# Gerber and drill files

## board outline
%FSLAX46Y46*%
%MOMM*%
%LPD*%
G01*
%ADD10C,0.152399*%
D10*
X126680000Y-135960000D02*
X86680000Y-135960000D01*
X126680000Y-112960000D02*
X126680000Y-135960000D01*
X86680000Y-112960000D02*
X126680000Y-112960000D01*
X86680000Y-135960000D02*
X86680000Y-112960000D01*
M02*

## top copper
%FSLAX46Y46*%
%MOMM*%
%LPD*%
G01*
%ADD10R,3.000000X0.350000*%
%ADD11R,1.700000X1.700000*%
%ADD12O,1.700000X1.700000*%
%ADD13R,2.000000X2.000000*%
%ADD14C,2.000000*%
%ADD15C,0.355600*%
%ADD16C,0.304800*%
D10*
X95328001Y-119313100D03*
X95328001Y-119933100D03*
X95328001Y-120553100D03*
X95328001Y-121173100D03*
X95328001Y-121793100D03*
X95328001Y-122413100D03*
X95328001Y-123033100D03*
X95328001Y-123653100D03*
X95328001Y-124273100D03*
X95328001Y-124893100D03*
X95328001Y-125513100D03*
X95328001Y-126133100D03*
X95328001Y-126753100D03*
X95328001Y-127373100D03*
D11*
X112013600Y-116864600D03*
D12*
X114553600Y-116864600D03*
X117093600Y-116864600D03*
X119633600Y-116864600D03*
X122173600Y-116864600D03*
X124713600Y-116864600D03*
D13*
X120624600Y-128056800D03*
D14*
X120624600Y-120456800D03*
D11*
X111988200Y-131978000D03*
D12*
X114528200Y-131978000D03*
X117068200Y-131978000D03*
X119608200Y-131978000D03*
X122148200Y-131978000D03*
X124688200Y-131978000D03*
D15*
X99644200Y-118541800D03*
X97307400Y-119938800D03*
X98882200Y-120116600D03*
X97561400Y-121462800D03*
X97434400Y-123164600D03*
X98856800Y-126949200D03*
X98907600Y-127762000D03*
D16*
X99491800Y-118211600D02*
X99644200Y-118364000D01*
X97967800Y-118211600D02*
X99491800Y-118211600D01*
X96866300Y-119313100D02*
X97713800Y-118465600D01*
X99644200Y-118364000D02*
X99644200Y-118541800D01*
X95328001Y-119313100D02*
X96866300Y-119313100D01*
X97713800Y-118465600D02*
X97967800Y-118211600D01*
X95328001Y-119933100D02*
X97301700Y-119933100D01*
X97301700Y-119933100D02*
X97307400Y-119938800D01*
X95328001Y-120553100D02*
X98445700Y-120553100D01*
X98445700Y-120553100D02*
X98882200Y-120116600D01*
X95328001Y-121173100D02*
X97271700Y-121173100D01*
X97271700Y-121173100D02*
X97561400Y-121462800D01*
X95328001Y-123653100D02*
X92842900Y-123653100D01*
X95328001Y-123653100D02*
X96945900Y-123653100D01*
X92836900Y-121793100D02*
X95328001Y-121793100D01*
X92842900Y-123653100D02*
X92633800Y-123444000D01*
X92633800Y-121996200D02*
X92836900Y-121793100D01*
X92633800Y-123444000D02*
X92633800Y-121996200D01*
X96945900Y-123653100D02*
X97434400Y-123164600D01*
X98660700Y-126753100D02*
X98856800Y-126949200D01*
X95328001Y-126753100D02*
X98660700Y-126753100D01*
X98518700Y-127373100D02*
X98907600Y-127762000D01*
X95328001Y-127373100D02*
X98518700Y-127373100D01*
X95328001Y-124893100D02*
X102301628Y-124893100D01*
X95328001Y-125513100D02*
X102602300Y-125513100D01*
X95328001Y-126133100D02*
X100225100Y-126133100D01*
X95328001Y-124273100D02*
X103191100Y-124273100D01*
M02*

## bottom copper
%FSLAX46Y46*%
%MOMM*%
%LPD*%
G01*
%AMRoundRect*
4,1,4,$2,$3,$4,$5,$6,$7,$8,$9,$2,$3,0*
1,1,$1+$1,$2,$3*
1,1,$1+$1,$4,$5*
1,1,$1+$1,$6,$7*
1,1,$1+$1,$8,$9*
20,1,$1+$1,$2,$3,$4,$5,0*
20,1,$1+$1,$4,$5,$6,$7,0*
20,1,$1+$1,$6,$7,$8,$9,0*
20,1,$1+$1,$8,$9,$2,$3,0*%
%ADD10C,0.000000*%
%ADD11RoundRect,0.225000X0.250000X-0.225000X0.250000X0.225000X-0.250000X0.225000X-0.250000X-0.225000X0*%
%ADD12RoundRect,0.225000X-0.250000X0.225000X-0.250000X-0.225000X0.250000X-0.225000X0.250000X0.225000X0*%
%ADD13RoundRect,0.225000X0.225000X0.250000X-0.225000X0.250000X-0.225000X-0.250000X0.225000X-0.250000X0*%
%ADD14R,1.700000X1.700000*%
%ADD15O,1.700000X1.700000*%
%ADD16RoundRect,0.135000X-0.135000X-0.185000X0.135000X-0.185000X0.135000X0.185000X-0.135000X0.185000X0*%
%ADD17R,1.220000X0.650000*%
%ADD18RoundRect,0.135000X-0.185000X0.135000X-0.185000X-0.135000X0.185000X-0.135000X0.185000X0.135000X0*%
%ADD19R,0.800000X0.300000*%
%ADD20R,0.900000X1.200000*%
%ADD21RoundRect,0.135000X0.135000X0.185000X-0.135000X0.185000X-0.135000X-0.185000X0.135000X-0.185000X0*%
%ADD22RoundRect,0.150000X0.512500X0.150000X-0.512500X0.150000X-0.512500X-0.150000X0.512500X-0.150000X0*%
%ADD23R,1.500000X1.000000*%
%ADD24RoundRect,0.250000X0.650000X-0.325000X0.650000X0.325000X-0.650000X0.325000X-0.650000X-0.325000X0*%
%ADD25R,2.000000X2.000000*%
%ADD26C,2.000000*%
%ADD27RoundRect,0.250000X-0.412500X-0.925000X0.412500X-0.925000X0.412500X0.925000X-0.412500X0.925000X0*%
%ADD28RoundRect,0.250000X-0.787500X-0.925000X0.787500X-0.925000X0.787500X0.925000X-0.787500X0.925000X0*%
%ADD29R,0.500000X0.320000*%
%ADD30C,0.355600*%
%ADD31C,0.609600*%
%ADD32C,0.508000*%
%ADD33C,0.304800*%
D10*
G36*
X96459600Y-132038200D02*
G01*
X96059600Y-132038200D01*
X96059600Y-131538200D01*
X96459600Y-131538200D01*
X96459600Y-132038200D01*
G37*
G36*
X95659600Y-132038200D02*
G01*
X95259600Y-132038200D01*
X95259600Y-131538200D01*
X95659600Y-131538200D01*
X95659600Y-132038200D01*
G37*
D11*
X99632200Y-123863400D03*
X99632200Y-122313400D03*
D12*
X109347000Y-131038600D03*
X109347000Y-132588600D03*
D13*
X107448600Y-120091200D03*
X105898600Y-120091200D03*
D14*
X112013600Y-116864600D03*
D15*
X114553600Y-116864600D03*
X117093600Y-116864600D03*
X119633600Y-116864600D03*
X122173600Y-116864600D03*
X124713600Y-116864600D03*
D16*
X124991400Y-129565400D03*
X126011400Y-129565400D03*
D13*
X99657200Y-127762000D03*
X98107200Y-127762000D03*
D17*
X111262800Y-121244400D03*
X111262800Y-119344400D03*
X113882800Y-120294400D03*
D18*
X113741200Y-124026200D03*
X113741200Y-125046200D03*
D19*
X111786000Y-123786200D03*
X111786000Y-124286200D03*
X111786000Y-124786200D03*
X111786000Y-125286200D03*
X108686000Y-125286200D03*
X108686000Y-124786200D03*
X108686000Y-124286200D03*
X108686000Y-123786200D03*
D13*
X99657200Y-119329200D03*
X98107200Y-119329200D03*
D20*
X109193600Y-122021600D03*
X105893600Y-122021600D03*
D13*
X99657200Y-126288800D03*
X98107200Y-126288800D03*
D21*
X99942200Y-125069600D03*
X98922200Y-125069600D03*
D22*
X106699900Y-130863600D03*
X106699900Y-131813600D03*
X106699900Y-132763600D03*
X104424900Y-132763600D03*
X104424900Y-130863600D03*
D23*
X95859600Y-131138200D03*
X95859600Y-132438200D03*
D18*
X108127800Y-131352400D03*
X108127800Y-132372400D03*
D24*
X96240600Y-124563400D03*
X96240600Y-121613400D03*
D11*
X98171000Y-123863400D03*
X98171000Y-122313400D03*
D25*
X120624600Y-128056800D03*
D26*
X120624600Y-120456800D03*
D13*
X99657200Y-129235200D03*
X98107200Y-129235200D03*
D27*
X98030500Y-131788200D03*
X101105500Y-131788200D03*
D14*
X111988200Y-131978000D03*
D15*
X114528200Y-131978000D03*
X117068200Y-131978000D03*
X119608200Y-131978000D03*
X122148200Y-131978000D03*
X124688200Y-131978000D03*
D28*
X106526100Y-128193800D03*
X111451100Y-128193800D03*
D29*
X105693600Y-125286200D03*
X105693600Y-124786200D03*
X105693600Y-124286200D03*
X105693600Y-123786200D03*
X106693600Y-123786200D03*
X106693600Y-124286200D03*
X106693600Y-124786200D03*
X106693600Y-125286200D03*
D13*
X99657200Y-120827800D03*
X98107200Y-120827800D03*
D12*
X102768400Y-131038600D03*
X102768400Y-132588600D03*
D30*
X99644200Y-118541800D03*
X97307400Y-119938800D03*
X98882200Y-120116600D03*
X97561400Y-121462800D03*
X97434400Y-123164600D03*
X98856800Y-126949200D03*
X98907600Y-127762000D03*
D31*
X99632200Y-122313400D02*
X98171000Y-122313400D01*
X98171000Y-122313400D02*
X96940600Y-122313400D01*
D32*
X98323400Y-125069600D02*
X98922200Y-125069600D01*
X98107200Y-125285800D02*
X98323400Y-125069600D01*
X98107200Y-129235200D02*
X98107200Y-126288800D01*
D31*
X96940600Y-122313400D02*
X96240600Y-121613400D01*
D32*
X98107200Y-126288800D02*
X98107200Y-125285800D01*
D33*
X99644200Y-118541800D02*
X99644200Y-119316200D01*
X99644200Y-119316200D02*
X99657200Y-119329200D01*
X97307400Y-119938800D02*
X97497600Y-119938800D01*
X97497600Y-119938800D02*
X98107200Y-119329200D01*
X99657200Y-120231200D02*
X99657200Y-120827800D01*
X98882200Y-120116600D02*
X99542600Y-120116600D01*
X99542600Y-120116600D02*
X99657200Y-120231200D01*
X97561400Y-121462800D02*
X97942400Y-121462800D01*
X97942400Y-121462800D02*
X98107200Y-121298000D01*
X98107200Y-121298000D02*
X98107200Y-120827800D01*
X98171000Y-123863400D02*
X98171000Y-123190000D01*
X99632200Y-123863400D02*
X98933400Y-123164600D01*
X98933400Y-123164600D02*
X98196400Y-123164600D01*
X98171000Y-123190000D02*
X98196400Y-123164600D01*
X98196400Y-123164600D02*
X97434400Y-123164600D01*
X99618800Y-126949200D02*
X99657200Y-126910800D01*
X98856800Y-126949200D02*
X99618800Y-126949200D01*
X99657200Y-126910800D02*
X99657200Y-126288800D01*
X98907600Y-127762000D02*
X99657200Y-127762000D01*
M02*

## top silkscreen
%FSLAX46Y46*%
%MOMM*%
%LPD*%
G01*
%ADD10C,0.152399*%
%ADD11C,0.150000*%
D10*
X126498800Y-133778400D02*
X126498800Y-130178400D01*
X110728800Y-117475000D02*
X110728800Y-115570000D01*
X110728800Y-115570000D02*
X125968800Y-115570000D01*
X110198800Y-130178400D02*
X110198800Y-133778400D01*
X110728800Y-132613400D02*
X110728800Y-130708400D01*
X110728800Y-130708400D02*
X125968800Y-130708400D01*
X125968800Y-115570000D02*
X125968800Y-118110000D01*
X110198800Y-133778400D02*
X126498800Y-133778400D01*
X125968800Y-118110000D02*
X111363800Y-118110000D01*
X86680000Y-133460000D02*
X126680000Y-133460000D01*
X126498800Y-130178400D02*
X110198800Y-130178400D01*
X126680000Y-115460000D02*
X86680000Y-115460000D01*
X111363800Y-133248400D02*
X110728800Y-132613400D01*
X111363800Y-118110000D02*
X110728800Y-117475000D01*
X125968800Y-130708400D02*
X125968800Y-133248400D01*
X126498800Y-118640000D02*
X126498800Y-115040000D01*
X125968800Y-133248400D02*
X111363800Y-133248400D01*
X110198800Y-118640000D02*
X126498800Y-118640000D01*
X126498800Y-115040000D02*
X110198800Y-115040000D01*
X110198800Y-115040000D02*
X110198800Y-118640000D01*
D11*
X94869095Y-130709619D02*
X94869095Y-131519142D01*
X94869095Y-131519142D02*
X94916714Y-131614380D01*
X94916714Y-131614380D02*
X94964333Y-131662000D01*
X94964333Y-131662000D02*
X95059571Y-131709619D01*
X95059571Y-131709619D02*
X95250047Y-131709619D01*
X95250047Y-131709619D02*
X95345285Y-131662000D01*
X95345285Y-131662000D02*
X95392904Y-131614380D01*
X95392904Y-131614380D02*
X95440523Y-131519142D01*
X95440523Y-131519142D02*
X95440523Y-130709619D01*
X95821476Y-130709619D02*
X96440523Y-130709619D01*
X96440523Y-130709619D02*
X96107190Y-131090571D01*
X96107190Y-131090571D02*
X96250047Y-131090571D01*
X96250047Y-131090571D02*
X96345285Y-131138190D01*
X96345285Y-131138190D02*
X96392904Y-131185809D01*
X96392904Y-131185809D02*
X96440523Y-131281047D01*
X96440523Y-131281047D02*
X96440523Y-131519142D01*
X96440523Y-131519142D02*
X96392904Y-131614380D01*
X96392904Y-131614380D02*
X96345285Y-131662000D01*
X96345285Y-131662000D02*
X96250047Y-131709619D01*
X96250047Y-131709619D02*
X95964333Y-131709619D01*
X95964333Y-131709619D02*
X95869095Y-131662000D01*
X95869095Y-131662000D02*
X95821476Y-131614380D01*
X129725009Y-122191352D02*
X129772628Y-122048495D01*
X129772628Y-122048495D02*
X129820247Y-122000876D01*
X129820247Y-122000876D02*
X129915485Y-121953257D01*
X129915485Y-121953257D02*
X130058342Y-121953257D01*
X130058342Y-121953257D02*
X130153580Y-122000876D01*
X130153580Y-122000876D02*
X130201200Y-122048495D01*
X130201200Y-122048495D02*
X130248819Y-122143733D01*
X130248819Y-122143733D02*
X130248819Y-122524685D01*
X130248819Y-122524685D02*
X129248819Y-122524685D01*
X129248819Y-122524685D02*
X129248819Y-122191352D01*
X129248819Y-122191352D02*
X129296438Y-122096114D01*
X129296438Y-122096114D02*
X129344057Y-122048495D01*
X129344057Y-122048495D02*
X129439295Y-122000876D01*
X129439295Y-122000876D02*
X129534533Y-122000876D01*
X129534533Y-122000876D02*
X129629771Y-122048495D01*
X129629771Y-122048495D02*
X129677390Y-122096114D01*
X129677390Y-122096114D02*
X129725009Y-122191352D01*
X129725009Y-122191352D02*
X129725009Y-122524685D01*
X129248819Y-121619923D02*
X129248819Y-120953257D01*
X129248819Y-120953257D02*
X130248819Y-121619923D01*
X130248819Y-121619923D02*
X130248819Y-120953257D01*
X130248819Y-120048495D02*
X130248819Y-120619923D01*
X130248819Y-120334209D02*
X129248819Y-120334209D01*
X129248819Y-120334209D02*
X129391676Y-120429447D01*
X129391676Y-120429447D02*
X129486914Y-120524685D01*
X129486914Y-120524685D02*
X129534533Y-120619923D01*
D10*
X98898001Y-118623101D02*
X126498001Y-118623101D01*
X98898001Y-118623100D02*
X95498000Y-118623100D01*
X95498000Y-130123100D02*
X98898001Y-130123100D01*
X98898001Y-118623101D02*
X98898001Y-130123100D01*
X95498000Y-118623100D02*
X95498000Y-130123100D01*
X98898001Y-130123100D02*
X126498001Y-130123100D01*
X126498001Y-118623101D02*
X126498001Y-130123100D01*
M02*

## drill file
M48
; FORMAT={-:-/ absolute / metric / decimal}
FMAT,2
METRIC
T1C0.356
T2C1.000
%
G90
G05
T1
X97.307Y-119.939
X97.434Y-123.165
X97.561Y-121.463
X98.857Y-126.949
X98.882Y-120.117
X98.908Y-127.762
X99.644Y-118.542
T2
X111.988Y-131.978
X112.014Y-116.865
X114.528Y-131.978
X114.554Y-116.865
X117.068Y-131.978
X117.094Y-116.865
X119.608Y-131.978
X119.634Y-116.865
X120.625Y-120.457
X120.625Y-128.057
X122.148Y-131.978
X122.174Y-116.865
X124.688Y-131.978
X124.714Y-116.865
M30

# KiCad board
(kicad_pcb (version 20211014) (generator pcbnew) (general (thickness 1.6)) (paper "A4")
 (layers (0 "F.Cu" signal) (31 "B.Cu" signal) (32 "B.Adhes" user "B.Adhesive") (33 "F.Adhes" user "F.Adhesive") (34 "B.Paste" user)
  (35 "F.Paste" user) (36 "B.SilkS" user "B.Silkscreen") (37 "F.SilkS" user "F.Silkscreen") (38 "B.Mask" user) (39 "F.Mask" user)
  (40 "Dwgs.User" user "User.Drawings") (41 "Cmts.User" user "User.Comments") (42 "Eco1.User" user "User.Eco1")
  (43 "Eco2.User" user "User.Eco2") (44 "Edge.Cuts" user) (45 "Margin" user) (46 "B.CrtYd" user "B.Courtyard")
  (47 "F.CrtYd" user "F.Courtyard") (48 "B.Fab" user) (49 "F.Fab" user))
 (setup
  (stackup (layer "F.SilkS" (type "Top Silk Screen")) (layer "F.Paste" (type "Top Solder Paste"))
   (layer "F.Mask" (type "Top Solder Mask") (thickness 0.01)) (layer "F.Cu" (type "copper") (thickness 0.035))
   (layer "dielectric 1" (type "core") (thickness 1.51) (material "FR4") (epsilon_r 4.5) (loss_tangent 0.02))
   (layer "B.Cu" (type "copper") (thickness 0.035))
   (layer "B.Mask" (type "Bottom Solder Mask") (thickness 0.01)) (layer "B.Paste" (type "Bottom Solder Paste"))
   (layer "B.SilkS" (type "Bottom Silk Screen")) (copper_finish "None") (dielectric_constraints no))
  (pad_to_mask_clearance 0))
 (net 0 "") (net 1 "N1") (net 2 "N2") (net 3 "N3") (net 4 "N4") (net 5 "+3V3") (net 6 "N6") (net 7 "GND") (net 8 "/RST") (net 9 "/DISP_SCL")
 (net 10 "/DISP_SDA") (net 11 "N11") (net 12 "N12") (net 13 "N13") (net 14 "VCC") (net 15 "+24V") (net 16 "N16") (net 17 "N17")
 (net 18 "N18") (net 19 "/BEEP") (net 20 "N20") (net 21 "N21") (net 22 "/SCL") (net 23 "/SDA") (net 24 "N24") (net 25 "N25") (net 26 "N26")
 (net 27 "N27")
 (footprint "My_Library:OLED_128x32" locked (layer "F.Cu") (at 98.898001 130.1231)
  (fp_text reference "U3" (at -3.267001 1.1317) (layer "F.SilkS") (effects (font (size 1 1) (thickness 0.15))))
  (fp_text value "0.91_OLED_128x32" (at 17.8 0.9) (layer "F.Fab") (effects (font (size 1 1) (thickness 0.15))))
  (fp_line (start 0 -11.499999) (end 27.6 -11.499999) (layer "F.SilkS") (width 0.152399))
  (fp_line (start 0 -11.5) (end -3.400001 -11.5) (layer "F.SilkS") (width 0.152399))
  (fp_line (start -3.400001 0) (end 0 0) (layer "F.SilkS") (width 0.152399))
  (fp_line (start 0 -11.499999) (end 0 0) (layer "F.SilkS") (width 0.152399))
  (fp_line (start -3.400001 -11.5) (end -3.400001 0) (layer "F.SilkS") (width 0.152399))
  (fp_line (start 0 0) (end 27.6 0) (layer "F.SilkS") (width 0.152399))
  (fp_line (start 27.6 -11.499999) (end 27.6 0) (layer "F.SilkS") (width 0.152399))
  (pad "1" smd rect locked (at -3.57 -10.81 90) (size 0.35 3) (layers "F.Cu" "F.Paste" "F.Mask") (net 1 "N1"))
  (pad "2" smd rect locked (at -3.57 -10.19 90) (size 0.35 3) (layers "F.Cu" "F.Paste" "F.Mask") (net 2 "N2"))
  (pad "3" smd rect locked (at -3.57 -9.57 90) (size 0.35 3) (layers "F.Cu" "F.Paste" "F.Mask") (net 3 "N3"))
  (pad "4" smd rect locked (at -3.57 -8.95 90) (size 0.35 3) (layers "F.Cu" "F.Paste" "F.Mask") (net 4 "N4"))
  (pad "5" smd rect locked (at -3.57 -8.33 90) (size 0.35 3) (layers "F.Cu" "F.Paste" "F.Mask") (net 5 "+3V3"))
  (pad "6" smd rect locked (at -3.57 -7.71 90) (size 0.35 3) (layers "F.Cu" "F.Paste" "F.Mask") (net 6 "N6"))
  (pad "7" smd rect locked (at -3.57 -7.09 90) (size 0.35 3) (layers "F.Cu" "F.Paste" "F.Mask") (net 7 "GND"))
  (pad "8" smd rect locked (at -3.57 -6.47 90) (size 0.35 3) (layers "F.Cu" "F.Paste" "F.Mask") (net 5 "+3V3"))
  (pad "9" smd rect locked (at -3.57 -5.85 90) (size 0.35 3) (layers "F.Cu" "F.Paste" "F.Mask") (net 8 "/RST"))
  (pad "10" smd rect locked (at -3.57 -5.23 90) (size 0.35 3) (layers "F.Cu" "F.Paste" "F.Mask") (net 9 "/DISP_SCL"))
  (pad "11" smd rect locked (at -3.57 -4.61 90) (size 0.35 3) (layers "F.Cu" "F.Paste" "F.Mask") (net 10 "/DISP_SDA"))
  (pad "12" smd rect locked (at -3.57 -3.99 90) (size 0.35 3) (layers "F.Cu" "F.Paste" "F.Mask") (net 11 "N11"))
  (pad "13" smd rect locked (at -3.57 -3.37 90) (size 0.35 3) (layers "F.Cu" "F.Paste" "F.Mask") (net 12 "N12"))
  (pad "14" smd rect locked (at -3.57 -2.75 90) (size 0.35 3) (layers "F.Cu" "F.Paste" "F.Mask") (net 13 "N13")))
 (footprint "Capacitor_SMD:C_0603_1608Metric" (layer "B.Cu") (at 99.6322 123.0884 90)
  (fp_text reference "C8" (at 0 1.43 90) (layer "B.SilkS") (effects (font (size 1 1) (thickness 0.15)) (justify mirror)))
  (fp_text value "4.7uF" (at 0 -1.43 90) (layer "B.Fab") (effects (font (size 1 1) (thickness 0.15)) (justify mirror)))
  (pad "1" smd roundrect (at -0.775 0 90) (size 0.9 0.95) (layers "B.Cu" "B.Paste" "B.Mask") (roundrect_rratio 0.25) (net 5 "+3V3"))
  (pad "2" smd roundrect (at 0.775 0 90) (size 0.9 0.95) (layers "B.Cu" "B.Paste" "B.Mask") (roundrect_rratio 0.25) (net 7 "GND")))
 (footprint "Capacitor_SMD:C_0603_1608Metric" (layer "B.Cu") (at 109.347 131.8136 -90)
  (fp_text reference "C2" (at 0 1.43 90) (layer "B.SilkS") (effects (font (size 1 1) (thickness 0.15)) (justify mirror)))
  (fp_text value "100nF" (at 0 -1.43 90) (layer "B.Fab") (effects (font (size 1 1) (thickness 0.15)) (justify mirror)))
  (pad "1" smd roundrect (at -0.775 0 270) (size 0.9 0.95) (layers "B.Cu" "B.Paste" "B.Mask") (roundrect_rratio 0.25) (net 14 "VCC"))
  (pad "2" smd roundrect (at 0.775 0 270) (size 0.9 0.95) (layers "B.Cu" "B.Paste" "B.Mask") (roundrect_rratio 0.25) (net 7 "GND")))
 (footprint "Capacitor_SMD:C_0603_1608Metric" (layer "B.Cu") (at 106.6736 120.0912 180)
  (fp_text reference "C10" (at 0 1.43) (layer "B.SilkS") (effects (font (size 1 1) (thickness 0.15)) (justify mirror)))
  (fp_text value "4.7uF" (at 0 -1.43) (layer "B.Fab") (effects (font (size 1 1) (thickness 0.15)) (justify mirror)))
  (pad "1" smd roundrect (at -0.775 0 180) (size 0.9 0.95) (layers "B.Cu" "B.Paste" "B.Mask") (roundrect_rratio 0.25) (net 7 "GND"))
  (pad "2" smd roundrect (at 0.775 0 180) (size 0.9 0.95) (layers "B.Cu" "B.Paste" "B.Mask") (roundrect_rratio 0.25) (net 8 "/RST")))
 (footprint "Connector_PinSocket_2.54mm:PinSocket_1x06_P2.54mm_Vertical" (layer "B.Cu") (at 112.0136 116.8646 -90)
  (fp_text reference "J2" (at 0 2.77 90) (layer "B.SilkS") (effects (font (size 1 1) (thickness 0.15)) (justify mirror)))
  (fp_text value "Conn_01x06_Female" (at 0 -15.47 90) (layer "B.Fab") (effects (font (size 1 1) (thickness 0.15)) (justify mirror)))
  (pad "1" thru_hole rect (at 0 0 270) (size 1.7 1.7) (drill 1) (layers *.Cu *.Mask) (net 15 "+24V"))
  (pad "2" thru_hole oval (at 0 -2.54 270) (size 1.7 1.7) (drill 1) (layers *.Cu *.Mask) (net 15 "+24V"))
  (pad "3" thru_hole oval (at 0 -5.08 270) (size 1.7 1.7) (drill 1) (layers *.Cu *.Mask) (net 7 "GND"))
  (pad "4" thru_hole oval (at 0 -7.62 270) (size 1.7 1.7) (drill 1) (layers *.Cu *.Mask) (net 7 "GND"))
  (pad "5" thru_hole oval (at 0 -10.16 270) (size 1.7 1.7) (drill 1) (layers *.Cu *.Mask) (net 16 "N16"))
  (pad "6" thru_hole oval (at 0 -12.7 270) (size 1.7 1.7) (drill 1) (layers *.Cu *.Mask) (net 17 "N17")))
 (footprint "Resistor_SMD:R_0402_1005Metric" (layer "B.Cu") (at 125.5014 129.5654)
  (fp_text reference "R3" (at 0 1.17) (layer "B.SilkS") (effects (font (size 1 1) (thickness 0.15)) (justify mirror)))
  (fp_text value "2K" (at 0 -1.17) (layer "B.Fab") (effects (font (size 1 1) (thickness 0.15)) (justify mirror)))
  (pad "1" smd roundrect (at -0.51 0) (size 0.54 0.64) (layers "B.Cu" "B.Paste" "B.Mask") (roundrect_rratio 0.25) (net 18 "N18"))
  (pad "2" smd roundrect (at 0.51 0) (size 0.54 0.64) (layers "B.Cu" "B.Paste" "B.Mask") (roundrect_rratio 0.25) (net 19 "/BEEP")))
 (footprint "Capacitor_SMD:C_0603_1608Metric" (layer "B.Cu") (at 98.8822 127.762 180)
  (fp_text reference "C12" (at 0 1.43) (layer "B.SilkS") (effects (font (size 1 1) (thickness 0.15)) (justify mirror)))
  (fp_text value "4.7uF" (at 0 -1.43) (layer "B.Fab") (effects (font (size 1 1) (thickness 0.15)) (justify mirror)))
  (pad "1" smd roundrect (at -0.775 0 180) (size 0.9 0.95) (layers "B.Cu" "B.Paste" "B.Mask") (roundrect_rratio 0.25) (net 13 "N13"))
  (pad "2" smd roundrect (at 0.775 0 180) (size 0.9 0.95) (layers "B.Cu" "B.Paste" "B.Mask") (roundrect_rratio 0.25) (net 7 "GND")))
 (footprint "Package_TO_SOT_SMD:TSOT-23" (layer "B.Cu") (at 112.5728 120.2944)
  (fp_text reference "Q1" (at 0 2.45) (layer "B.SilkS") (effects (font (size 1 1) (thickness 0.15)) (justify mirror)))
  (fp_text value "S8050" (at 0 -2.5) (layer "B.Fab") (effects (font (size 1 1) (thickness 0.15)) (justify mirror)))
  (pad "1" smd rect (at -1.31 0.95) (size 1.22 0.65) (layers "B.Cu" "B.Paste" "B.Mask") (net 7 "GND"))
  (pad "2" smd rect (at -1.31 -0.95) (size 1.22 0.65) (layers "B.Cu" "B.Paste" "B.Mask") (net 18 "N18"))
  (pad "3" smd rect (at 1.31 0) (size 1.22 0.65) (layers "B.Cu" "B.Paste" "B.Mask") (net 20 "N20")))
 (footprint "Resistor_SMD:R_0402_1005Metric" (layer "B.Cu") (at 113.7412 124.5362 -90)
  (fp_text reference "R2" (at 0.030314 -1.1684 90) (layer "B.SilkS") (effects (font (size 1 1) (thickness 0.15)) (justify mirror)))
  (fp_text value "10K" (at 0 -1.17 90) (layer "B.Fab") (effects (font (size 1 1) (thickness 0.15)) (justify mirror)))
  (pad "1" smd roundrect (at -0.51 0 270) (size 0.54 0.64) (layers "B.Cu" "B.Paste" "B.Mask") (roundrect_rratio 0.25) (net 14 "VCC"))
  (pad "2" smd roundrect (at 0.51 0 270) (size 0.54 0.64) (layers "B.Cu" "B.Paste" "B.Mask") (roundrect_rratio 0.25) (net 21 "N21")))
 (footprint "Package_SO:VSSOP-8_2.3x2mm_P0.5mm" (layer "B.Cu") (at 110.236 124.5362 180)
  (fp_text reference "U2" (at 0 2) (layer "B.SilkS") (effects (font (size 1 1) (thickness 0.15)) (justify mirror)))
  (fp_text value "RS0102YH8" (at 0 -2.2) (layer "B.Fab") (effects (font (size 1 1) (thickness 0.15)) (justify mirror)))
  (pad "1" smd rect (at -1.55 0.75 270) (size 0.3 0.8) (layers "B.Cu" "B.Paste" "B.Mask") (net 14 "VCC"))
  (pad "2" smd rect (at -1.55 0.25 270) (size 0.3 0.8) (layers "B.Cu" "B.Paste" "B.Mask") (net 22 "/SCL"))
  (pad "3" smd rect (at -1.55 -0.25 270) (size 0.3 0.8) (layers "B.Cu" "B.Paste" "B.Mask") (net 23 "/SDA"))
  (pad "4" smd rect (at -1.55 -0.75 270) (size 0.3 0.8) (layers "B.Cu" "B.Paste" "B.Mask") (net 21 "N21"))
  (pad "5" smd rect (at 1.55 -0.75 270) (size 0.3 0.8) (layers "B.Cu" "B.Paste" "B.Mask") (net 7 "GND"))
  (pad "6" smd rect (at 1.55 -0.25 270) (size 0.3 0.8) (layers "B.Cu" "B.Paste" "B.Mask") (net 10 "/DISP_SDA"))
  (pad "7" smd rect (at 1.55 0.25 270) (size 0.3 0.8) (layers "B.Cu" "B.Paste" "B.Mask") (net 9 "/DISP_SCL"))
  (pad "8" smd rect (at 1.55 0.75 270) (size 0.3 0.8) (layers "B.Cu" "B.Paste" "B.Mask") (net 5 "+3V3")))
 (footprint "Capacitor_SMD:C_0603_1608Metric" (layer "B.Cu") (at 98.8822 119.3292 180)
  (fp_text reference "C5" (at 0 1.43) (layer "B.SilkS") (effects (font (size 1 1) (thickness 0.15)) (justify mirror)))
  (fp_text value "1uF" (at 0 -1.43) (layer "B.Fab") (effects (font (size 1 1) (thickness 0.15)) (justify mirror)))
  (pad "1" smd roundrect (at -0.775 0 180) (size 0.9 0.95) (layers "B.Cu" "B.Paste" "B.Mask") (roundrect_rratio 0.25) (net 1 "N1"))
  (pad "2" smd roundrect (at 0.775 0 180) (size 0.9 0.95) (layers "B.Cu" "B.Paste" "B.Mask") (roundrect_rratio 0.25) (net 2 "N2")))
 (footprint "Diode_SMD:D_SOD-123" (layer "B.Cu") (at 107.5436 122.0216 180)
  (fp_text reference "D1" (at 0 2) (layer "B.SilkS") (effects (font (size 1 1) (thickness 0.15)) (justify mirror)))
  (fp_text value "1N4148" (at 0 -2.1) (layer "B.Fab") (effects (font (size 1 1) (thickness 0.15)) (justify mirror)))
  (pad "1" smd rect (at -1.65 0 180) (size 0.9 1.2) (layers "B.Cu" "B.Paste" "B.Mask") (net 5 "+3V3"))
  (pad "2" smd rect (at 1.65 0 180) (size 0.9 1.2) (layers "B.Cu" "B.Paste" "B.Mask") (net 8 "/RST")))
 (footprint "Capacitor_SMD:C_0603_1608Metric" (layer "B.Cu") (at 98.8822 126.2888 180)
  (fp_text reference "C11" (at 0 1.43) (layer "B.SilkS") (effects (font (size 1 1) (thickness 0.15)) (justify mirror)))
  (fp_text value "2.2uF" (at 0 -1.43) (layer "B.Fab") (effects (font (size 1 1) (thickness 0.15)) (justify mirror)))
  (pad "1" smd roundrect (at -0.775 0 180) (size 0.9 0.95) (layers "B.Cu" "B.Paste" "B.Mask") (roundrect_rratio 0.25) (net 12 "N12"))
  (pad "2" smd roundrect (at 0.775 0 180) (size 0.9 0.95) (layers "B.Cu" "B.Paste" "B.Mask") (roundrect_rratio 0.25) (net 7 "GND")))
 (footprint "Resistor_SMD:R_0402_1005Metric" (layer "B.Cu") (at 99.4322 125.0696 180)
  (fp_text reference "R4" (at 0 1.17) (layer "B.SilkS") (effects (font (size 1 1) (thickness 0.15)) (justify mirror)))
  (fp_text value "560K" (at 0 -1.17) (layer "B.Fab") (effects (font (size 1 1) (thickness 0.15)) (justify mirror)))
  (pad "1" smd roundrect (at -0.51 0 180) (size 0.54 0.64) (layers "B.Cu" "B.Paste" "B.Mask") (roundrect_rratio 0.25) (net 11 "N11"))
  (pad "2" smd roundrect (at 0.51 0 180) (size 0.54 0.64) (layers "B.Cu" "B.Paste" "B.Mask") (roundrect_rratio 0.25) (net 7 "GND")))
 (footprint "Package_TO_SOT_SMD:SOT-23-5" (layer "B.Cu") (at 105.5624 131.8136 180)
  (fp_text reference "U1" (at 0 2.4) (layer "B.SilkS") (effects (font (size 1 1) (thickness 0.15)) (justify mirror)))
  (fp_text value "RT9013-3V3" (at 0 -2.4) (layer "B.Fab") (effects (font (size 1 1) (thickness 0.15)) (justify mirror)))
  (pad "1" smd roundrect (at -1.1375 0.95 180) (size 1.325 0.6) (layers "B.Cu" "B.Paste" "B.Mask") (roundrect_rratio 0.25) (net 14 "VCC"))
  (pad "2" smd roundrect (at -1.1375 0 180) (size 1.325 0.6) (layers "B.Cu" "B.Paste" "B.Mask") (roundrect_rratio 0.25) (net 7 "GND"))
  (pad "3" smd roundrect (at -1.1375 -0.95 180) (size 1.325 0.6) (layers "B.Cu" "B.Paste" "B.Mask") (roundrect_rratio 0.25) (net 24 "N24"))
  (pad "4" smd roundrect (at 1.1375 -0.95 180) (size 1.325 0.6) (layers "B.Cu" "B.Paste" "B.Mask") (roundrect_rratio 0.25) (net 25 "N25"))
  (pad "5" smd roundrect (at 1.1375 0.95 180) (size 1.325 0.6) (layers "B.Cu" "B.Paste" "B.Mask") (roundrect_rratio 0.25) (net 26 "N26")))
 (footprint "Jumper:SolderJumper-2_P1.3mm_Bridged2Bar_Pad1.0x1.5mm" (layer "B.Cu") (at 95.8596 131.7882 -90)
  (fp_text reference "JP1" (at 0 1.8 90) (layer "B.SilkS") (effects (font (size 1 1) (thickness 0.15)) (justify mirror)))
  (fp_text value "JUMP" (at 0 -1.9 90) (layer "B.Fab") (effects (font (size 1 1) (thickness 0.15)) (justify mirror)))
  (fp_poly (pts (xy -0.25 -0.2) (xy 0.25 -0.2) (xy 0.25 -0.6) (xy -0.25 -0.6)) (layer "B.Cu") (width 0) (fill solid))
  (fp_poly (pts (xy -0.25 0.6) (xy 0.25 0.6) (xy 0.25 0.2) (xy -0.25 0.2)) (layer "B.Cu") (width 0) (fill solid))
  (pad "1" smd rect (at -0.65 0 270) (size 1 1.5) (layers "B.Cu" "B.Mask") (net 5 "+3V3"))
  (pad "2" smd rect (at 0.65 0 270) (size 1 1.5) (layers "B.Cu" "B.Mask") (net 26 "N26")))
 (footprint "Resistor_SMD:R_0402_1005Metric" (layer "B.Cu") (at 108.1278 131.8624 -90)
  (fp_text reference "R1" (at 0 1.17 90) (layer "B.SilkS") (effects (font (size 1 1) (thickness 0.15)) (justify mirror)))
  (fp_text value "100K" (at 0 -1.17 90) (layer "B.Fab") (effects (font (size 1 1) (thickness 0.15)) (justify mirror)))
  (pad "1" smd roundrect (at -0.51 0 270) (size 0.54 0.64) (layers "B.Cu" "B.Paste" "B.Mask") (roundrect_rratio 0.25) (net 14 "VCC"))
  (pad "2" smd roundrect (at 0.51 0 270) (size 0.54 0.64) (layers "B.Cu" "B.Paste" "B.Mask") (roundrect_rratio 0.25) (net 24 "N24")))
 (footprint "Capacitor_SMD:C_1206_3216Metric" (layer "B.Cu") (at 96.2406 123.0884 90)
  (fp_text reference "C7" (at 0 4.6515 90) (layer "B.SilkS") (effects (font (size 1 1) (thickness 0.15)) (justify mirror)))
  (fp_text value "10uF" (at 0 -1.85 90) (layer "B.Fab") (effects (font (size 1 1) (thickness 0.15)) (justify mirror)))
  (pad "1" smd roundrect (at -1.475 0 90) (size 1.15 1.8) (layers "B.Cu" "B.Paste" "B.Mask") (roundrect_rratio 0.217391) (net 14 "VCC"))
  (pad "2" smd roundrect (at 1.475 0 90) (size 1.15 1.8) (layers "B.Cu" "B.Paste" "B.Mask") (roundrect_rratio 0.217391) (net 7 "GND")))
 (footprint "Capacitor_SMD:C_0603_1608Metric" (layer "B.Cu") (at 98.171 123.0884 90)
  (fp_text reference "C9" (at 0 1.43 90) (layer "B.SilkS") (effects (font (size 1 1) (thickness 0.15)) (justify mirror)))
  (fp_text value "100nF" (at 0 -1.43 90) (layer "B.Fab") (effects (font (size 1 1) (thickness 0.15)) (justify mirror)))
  (pad "1" smd roundrect (at -0.775 0 90) (size 0.9 0.95) (layers "B.Cu" "B.Paste" "B.Mask") (roundrect_rratio 0.25) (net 5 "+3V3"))
  (pad "2" smd roundrect (at 0.775 0 90) (size 0.9 0.95) (layers "B.Cu" "B.Paste" "B.Mask") (roundrect_rratio 0.25) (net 7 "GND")))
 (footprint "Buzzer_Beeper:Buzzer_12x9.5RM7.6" (layer "B.Cu") (at 120.6246 128.0568 90)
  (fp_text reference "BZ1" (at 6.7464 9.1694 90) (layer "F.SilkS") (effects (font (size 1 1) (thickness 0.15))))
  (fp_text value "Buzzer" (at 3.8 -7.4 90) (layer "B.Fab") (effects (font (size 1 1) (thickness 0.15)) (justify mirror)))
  (pad "1" thru_hole rect (at 0 0 90) (size 2 2) (drill 1) (layers *.Cu *.Mask) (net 14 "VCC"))
  (pad "2" thru_hole circle (at 7.6 0 90) (size 2 2) (drill 1) (layers *.Cu *.Mask) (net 20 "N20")))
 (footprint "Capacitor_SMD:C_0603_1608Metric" (layer "B.Cu") (at 98.8822 129.2352 180)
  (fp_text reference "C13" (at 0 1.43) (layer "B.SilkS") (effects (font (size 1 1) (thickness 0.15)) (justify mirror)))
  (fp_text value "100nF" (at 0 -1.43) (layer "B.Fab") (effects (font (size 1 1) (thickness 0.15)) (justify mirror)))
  (pad "1" smd roundrect (at -0.775 0 180) (size 0.9 0.95) (layers "B.Cu" "B.Paste" "B.Mask") (roundrect_rratio 0.25) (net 13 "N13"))
  (pad "2" smd roundrect (at 0.775 0 180) (size 0.9 0.95) (layers "B.Cu" "B.Paste" "B.Mask") (roundrect_rratio 0.25) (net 7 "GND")))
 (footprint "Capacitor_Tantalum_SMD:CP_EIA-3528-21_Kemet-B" (layer "B.Cu") (at 99.568 131.7882)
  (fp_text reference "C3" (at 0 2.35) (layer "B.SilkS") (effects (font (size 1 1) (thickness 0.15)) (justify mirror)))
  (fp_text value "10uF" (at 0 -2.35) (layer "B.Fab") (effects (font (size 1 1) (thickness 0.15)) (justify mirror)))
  (pad "1" smd roundrect (at -1.5375 0) (size 1.325 2.35) (layers "B.Cu" "B.Paste" "B.Mask") (roundrect_rratio 0.188679) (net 26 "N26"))
  (pad "2" smd roundrect (at 1.5375 0) (size 1.325 2.35) (layers "B.Cu" "B.Paste" "B.Mask") (roundrect_rratio 0.188679) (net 7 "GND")))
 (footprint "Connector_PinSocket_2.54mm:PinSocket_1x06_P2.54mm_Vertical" (layer "B.Cu") (at 111.9882 131.978 -90)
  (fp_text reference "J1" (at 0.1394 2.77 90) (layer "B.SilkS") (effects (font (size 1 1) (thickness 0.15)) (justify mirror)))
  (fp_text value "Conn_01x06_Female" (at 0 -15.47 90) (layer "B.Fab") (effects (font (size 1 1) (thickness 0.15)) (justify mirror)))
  (pad "1" thru_hole rect (at 0 0 270) (size 1.7 1.7) (drill 1) (layers *.Cu *.Mask) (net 14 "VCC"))
  (pad "2" thru_hole oval (at 0 -2.54 270) (size 1.7 1.7) (drill 1) (layers *.Cu *.Mask) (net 23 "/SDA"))
  (pad "3" thru_hole oval (at 0 -5.08 270) (size 1.7 1.7) (drill 1) (layers *.Cu *.Mask) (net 22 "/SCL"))
  (pad "4" thru_hole oval (at 0 -7.62 270) (size 1.7 1.7) (drill 1) (layers *.Cu *.Mask) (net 8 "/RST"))
  (pad "5" thru_hole oval (at 0 -10.16 270) (size 1.7 1.7) (drill 1) (layers *.Cu *.Mask) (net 7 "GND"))
  (pad "6" thru_hole oval (at 0 -12.7 270) (size 1.7 1.7) (drill 1) (layers *.Cu *.Mask) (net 19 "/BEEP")))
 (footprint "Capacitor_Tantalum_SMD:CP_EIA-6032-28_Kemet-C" (layer "B.Cu") (at 108.9886 128.1938)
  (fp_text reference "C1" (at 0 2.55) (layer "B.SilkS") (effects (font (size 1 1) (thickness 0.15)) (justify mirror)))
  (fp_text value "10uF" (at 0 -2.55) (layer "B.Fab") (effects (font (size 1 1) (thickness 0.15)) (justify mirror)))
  (pad "1" smd roundrect (at -2.4625 0) (size 2.075 2.35) (layers "B.Cu" "B.Paste" "B.Mask") (roundrect_rratio 0.120482) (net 14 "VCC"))
  (pad "2" smd roundrect (at 2.4625 0) (size 2.075 2.35) (layers "B.Cu" "B.Paste" "B.Mask") (roundrect_rratio 0.120482) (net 7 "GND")))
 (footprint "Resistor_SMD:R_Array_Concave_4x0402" (layer "B.Cu") (at 106.1936 124.5362)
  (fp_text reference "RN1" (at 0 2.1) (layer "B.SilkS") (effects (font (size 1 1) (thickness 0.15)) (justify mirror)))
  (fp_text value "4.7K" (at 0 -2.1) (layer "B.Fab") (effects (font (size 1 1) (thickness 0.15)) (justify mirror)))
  (pad "1" smd rect (at -0.5 0.75) (size 0.5 0.32) (layers "B.Cu" "B.Paste" "B.Mask") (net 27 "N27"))
  (pad "2" smd rect (at -0.5 0.25) (size 0.5 0.32) (layers "B.Cu" "B.Paste" "B.Mask") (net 10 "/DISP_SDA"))
  (pad "3" smd rect (at -0.5 -0.25) (size 0.5 0.32) (layers "B.Cu" "B.Paste" "B.Mask") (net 9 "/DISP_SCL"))
  (pad "4" smd rect (at -0.5 -0.75) (size 0.5 0.32) (layers "B.Cu" "B.Paste" "B.Mask") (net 8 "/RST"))
  (pad "5" smd rect (at 0.5 -0.75) (size 0.5 0.32) (layers "B.Cu" "B.Paste" "B.Mask") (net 5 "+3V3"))
  (pad "6" smd rect (at 0.5 -0.25) (size 0.5 0.32) (layers "B.Cu" "B.Paste" "B.Mask") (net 5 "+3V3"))
  (pad "7" smd rect (at 0.5 0.25) (size 0.5 0.32) (layers "B.Cu" "B.Paste" "B.Mask") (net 5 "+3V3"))
  (pad "8" smd rect (at 0.5 0.75) (size 0.5 0.32) (layers "B.Cu" "B.Paste" "B.Mask") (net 5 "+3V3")))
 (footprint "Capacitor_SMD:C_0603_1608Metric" (layer "B.Cu") (at 98.8822 120.8278 180)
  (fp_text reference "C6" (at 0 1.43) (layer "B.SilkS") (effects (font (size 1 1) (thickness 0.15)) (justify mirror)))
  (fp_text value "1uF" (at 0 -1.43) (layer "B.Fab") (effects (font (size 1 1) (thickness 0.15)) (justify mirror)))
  (pad "1" smd roundrect (at -0.775 0 180) (size 0.9 0.95) (layers "B.Cu" "B.Paste" "B.Mask") (roundrect_rratio 0.25) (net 3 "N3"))
  (pad "2" smd roundrect (at 0.775 0 180) (size 0.9 0.95) (layers "B.Cu" "B.Paste" "B.Mask") (roundrect_rratio 0.25) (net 4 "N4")))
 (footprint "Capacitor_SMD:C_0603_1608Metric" (layer "B.Cu") (at 102.7684 131.8136 -90)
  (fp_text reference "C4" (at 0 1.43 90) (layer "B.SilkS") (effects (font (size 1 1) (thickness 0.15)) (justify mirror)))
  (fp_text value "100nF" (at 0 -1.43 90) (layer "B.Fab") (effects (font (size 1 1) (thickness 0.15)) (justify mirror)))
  (pad "1" smd roundrect (at -0.775 0 270) (size 0.9 0.95) (layers "B.Cu" "B.Paste" "B.Mask") (roundrect_rratio 0.25) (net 26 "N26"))
  (pad "2" smd roundrect (at 0.775 0 270) (size 0.9 0.95) (layers "B.Cu" "B.Paste" "B.Mask") (roundrect_rratio 0.25) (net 7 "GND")))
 (gr_line (start 126.4988 133.7784) (end 126.4988 130.1784) (layer "F.SilkS") (width 0.152399))
 (gr_line (start 110.7288 117.475) (end 110.7288 115.57) (layer "F.SilkS") (width 0.152399))
 (gr_line (start 110.7288 115.57) (end 125.9688 115.57) (layer "F.SilkS") (width 0.152399))
 (gr_line (start 110.1988 130.1784) (end 110.1988 133.7784) (layer "F.SilkS") (width 0.152399))
 (gr_line (start 110.7288 132.6134) (end 110.7288 130.7084) (layer "F.SilkS") (width 0.152399))
 (gr_line (start 110.7288 130.7084) (end 125.9688 130.7084) (layer "F.SilkS") (width 0.152399))
 (gr_line (start 125.9688 115.57) (end 125.9688 118.11) (layer "F.SilkS") (width 0.152399))
 (gr_line (start 110.1988 133.7784) (end 126.4988 133.7784) (layer "F.SilkS") (width 0.152399))
 (gr_line (start 125.9688 118.11) (end 111.3638 118.11) (layer "F.SilkS") (width 0.152399))
 (gr_line (start 86.68 133.46) (end 126.68 133.46) (layer "F.SilkS") (width 0.152399))
 (gr_line (start 126.4988 130.1784) (end 110.1988 130.1784) (layer "F.SilkS") (width 0.152399))
 (gr_line (start 126.68 115.46) (end 86.68 115.46) (layer "F.SilkS") (width 0.152399))
 (gr_line (start 111.3638 133.2484) (end 110.7288 132.6134) (layer "F.SilkS") (width 0.152399))
 (gr_line (start 111.3638 118.11) (end 110.7288 117.475) (layer "F.SilkS") (width 0.152399))
 (gr_line (start 125.9688 130.7084) (end 125.9688 133.2484) (layer "F.SilkS") (width 0.152399))
 (gr_line (start 126.4988 118.64) (end 126.4988 115.04) (layer "F.SilkS") (width 0.152399))
 (gr_line (start 125.9688 133.2484) (end 111.3638 133.2484) (layer "F.SilkS") (width 0.152399))
 (gr_line (start 110.1988 118.64) (end 126.4988 118.64) (layer "F.SilkS") (width 0.152399))
 (gr_line (start 126.4988 115.04) (end 110.1988 115.04) (layer "F.SilkS") (width 0.152399))
 (gr_line (start 110.1988 115.04) (end 110.1988 118.64) (layer "F.SilkS") (width 0.152399))
 (gr_line (start 126.68 135.96) (end 86.68 135.96) (layer "Edge.Cuts") (width 0.152399))
 (gr_line (start 126.68 112.96) (end 126.68 135.96) (layer "Edge.Cuts") (width 0.152399))
 (gr_line (start 86.68 112.96) (end 126.68 112.96) (layer "Edge.Cuts") (width 0.152399))
 (gr_line (start 86.68 135.96) (end 86.68 112.96) (layer "Edge.Cuts") (width 0.152399))
 (segment (start 99.6322 122.3134) (end 98.171 122.3134) (width 0.6096) (layer "B.Cu") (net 7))
 (segment (start 98.171 122.3134) (end 96.9406 122.3134) (width 0.6096) (layer "B.Cu") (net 7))
 (segment (start 98.3234 125.0696) (end 98.9222 125.0696) (width 0.508) (layer "B.Cu") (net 7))
 (segment (start 98.1072 125.2858) (end 98.3234 125.0696) (width 0.508) (layer "B.Cu") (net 7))
 (segment (start 98.1072 129.2352) (end 98.1072 126.2888) (width 0.508) (layer "B.Cu") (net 7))
 (segment (start 96.9406 122.3134) (end 96.2406 121.6134) (width 0.6096) (layer "B.Cu") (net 7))
 (segment (start 98.1072 126.2888) (end 98.1072 125.2858) (width 0.508) (layer "B.Cu") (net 7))
 (segment (start 99.4918 118.2116) (end 99.6442 118.364) (width 0.3048) (layer "F.Cu") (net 1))
 (segment (start 97.9678 118.2116) (end 99.4918 118.2116) (width 0.3048) (layer "F.Cu") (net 1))
 (segment (start 96.8663 119.3131) (end 97.7138 118.4656) (width 0.3048) (layer "F.Cu") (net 1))
 (segment (start 99.6442 118.364) (end 99.6442 118.5418) (width 0.3048) (layer "F.Cu") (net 1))
 (segment (start 95.328001 119.3131) (end 96.8663 119.3131) (width 0.3048) (layer "F.Cu") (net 1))
 (segment (start 97.7138 118.4656) (end 97.9678 118.2116) (width 0.3048) (layer "F.Cu") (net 1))
 (via (at 99.6442 118.5418) (size 0.3556) (drill 0.3556) (layers "F.Cu" "B.Cu") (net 1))
 (segment (start 99.6442 118.5418) (end 99.6442 119.3162) (width 0.3048) (layer "B.Cu") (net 1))
 (segment (start 99.6442 119.3162) (end 99.6572 119.3292) (width 0.3048) (layer "B.Cu") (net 1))
 (segment (start 95.328001 119.9331) (end 97.3017 119.9331) (width 0.3048) (layer "F.Cu") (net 2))
 (segment (start 97.3017 119.9331) (end 97.3074 119.9388) (width 0.3048) (layer "F.Cu") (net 2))
 (via (at 97.3074 119.9388) (size 0.3556) (drill 0.3556) (layers "F.Cu" "B.Cu") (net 2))
 (segment (start 97.3074 119.9388) (end 97.4976 119.9388) (width 0.3048) (layer "B.Cu") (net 2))
 (segment (start 97.4976 119.9388) (end 98.1072 119.3292) (width 0.3048) (layer "B.Cu") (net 2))
 (segment (start 95.328001 120.5531) (end 98.4457 120.5531) (width 0.3048) (layer "F.Cu") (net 3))
 (segment (start 98.4457 120.5531) (end 98.8822 120.1166) (width 0.3048) (layer "F.Cu") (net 3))
 (via (at 98.8822 120.1166) (size 0.3556) (drill 0.3556) (layers "F.Cu" "B.Cu") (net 3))
 (segment (start 99.6572 120.2312) (end 99.6572 120.8278) (width 0.3048) (layer "B.Cu") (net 3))
 (segment (start 98.8822 120.1166) (end 99.5426 120.1166) (width 0.3048) (layer "B.Cu") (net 3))
 (segment (start 99.5426 120.1166) (end 99.6572 120.2312) (width 0.3048) (layer "B.Cu") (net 3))
 (segment (start 95.328001 121.1731) (end 97.2717 121.1731) (width 0.3048) (layer "F.Cu") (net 4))
 (segment (start 97.2717 121.1731) (end 97.5614 121.4628) (width 0.3048) (layer "F.Cu") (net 4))
 (via (at 97.5614 121.4628) (size 0.3556) (drill 0.3556) (layers "F.Cu" "B.Cu") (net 4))
 (segment (start 97.5614 121.4628) (end 97.9424 121.4628) (width 0.3048) (layer "B.Cu") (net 4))
 (segment (start 97.9424 121.4628) (end 98.1072 121.298) (width 0.3048) (layer "B.Cu") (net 4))
 (segment (start 98.1072 121.298) (end 98.1072 120.8278) (width 0.3048) (layer "B.Cu") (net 4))
 (segment (start 95.328001 123.6531) (end 92.8429 123.6531) (width 0.3048) (layer "F.Cu") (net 5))
 (segment (start 95.328001 123.6531) (end 96.9459 123.6531) (width 0.3048) (layer "F.Cu") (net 5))
 (segment (start 92.8369 121.7931) (end 95.328001 121.7931) (width 0.3048) (layer "F.Cu") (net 5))
 (segment (start 92.8429 123.6531) (end 92.6338 123.444) (width 0.3048) (layer "F.Cu") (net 5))
 (segment (start 92.6338 121.9962) (end 92.8369 121.7931) (width 0.3048) (layer "F.Cu") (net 5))
 (segment (start 92.6338 123.444) (end 92.6338 121.9962) (width 0.3048) (layer "F.Cu") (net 5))
 (segment (start 96.9459 123.6531) (end 97.4344 123.1646) (width 0.3048) (layer "F.Cu") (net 5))
 (via (at 97.4344 123.1646) (size 0.3556) (drill 0.3556) (layers "F.Cu" "B.Cu") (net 5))
 (segment (start 98.171 123.8634) (end 98.171 123.19) (width 0.3048) (layer "B.Cu") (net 5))
 (segment (start 99.6322 123.8634) (end 98.9334 123.1646) (width 0.3048) (layer "B.Cu") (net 5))
 (segment (start 98.9334 123.1646) (end 98.1964 123.1646) (width 0.3048) (layer "B.Cu") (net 5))
 (segment (start 98.171 123.19) (end 98.1964 123.1646) (width 0.3048) (layer "B.Cu") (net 5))
 (segment (start 98.1964 123.1646) (end 97.4344 123.1646) (width 0.3048) (layer "B.Cu") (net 5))
 (segment (start 98.6607 126.7531) (end 98.8568 126.9492) (width 0.3048) (layer "F.Cu") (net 12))
 (segment (start 95.328001 126.7531) (end 98.6607 126.7531) (width 0.3048) (layer "F.Cu") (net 12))
 (via (at 98.8568 126.9492) (size 0.3556) (drill 0.3556) (layers "F.Cu" "B.Cu") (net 12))
 (segment (start 99.6188 126.9492) (end 99.6572 126.9108) (width 0.3048) (layer "B.Cu") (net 12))
 (segment (start 98.8568 126.9492) (end 99.6188 126.9492) (width 0.3048) (layer "B.Cu") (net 12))
 (segment (start 99.6572 126.9108) (end 99.6572 126.2888) (width 0.3048) (layer "B.Cu") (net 12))
 (segment (start 98.5187 127.3731) (end 98.9076 127.762) (width 0.3048) (layer "F.Cu") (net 13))
 (segment (start 95.328001 127.3731) (end 98.5187 127.3731) (width 0.3048) (layer "F.Cu") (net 13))
 (via (at 98.9076 127.762) (size 0.3556) (drill 0.3556) (layers "F.Cu" "B.Cu") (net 13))
 (segment (start 98.9076 127.762) (end 99.6572 127.762) (width 0.3048) (layer "B.Cu") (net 13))
 (segment (start 95.328001 124.8931) (end 102.301628 124.8931) (width 0.3048) (layer "F.Cu") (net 9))
 (segment (start 95.328001 125.5131) (end 102.6023 125.5131) (width 0.3048) (layer "F.Cu") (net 10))
 (segment (start 95.328001 126.1331) (end 100.2251 126.1331) (width 0.3048) (layer "F.Cu") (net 11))
 (segment (start 95.328001 124.2731) (end 103.1911 124.2731) (width 0.3048) (layer "F.Cu") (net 8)))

